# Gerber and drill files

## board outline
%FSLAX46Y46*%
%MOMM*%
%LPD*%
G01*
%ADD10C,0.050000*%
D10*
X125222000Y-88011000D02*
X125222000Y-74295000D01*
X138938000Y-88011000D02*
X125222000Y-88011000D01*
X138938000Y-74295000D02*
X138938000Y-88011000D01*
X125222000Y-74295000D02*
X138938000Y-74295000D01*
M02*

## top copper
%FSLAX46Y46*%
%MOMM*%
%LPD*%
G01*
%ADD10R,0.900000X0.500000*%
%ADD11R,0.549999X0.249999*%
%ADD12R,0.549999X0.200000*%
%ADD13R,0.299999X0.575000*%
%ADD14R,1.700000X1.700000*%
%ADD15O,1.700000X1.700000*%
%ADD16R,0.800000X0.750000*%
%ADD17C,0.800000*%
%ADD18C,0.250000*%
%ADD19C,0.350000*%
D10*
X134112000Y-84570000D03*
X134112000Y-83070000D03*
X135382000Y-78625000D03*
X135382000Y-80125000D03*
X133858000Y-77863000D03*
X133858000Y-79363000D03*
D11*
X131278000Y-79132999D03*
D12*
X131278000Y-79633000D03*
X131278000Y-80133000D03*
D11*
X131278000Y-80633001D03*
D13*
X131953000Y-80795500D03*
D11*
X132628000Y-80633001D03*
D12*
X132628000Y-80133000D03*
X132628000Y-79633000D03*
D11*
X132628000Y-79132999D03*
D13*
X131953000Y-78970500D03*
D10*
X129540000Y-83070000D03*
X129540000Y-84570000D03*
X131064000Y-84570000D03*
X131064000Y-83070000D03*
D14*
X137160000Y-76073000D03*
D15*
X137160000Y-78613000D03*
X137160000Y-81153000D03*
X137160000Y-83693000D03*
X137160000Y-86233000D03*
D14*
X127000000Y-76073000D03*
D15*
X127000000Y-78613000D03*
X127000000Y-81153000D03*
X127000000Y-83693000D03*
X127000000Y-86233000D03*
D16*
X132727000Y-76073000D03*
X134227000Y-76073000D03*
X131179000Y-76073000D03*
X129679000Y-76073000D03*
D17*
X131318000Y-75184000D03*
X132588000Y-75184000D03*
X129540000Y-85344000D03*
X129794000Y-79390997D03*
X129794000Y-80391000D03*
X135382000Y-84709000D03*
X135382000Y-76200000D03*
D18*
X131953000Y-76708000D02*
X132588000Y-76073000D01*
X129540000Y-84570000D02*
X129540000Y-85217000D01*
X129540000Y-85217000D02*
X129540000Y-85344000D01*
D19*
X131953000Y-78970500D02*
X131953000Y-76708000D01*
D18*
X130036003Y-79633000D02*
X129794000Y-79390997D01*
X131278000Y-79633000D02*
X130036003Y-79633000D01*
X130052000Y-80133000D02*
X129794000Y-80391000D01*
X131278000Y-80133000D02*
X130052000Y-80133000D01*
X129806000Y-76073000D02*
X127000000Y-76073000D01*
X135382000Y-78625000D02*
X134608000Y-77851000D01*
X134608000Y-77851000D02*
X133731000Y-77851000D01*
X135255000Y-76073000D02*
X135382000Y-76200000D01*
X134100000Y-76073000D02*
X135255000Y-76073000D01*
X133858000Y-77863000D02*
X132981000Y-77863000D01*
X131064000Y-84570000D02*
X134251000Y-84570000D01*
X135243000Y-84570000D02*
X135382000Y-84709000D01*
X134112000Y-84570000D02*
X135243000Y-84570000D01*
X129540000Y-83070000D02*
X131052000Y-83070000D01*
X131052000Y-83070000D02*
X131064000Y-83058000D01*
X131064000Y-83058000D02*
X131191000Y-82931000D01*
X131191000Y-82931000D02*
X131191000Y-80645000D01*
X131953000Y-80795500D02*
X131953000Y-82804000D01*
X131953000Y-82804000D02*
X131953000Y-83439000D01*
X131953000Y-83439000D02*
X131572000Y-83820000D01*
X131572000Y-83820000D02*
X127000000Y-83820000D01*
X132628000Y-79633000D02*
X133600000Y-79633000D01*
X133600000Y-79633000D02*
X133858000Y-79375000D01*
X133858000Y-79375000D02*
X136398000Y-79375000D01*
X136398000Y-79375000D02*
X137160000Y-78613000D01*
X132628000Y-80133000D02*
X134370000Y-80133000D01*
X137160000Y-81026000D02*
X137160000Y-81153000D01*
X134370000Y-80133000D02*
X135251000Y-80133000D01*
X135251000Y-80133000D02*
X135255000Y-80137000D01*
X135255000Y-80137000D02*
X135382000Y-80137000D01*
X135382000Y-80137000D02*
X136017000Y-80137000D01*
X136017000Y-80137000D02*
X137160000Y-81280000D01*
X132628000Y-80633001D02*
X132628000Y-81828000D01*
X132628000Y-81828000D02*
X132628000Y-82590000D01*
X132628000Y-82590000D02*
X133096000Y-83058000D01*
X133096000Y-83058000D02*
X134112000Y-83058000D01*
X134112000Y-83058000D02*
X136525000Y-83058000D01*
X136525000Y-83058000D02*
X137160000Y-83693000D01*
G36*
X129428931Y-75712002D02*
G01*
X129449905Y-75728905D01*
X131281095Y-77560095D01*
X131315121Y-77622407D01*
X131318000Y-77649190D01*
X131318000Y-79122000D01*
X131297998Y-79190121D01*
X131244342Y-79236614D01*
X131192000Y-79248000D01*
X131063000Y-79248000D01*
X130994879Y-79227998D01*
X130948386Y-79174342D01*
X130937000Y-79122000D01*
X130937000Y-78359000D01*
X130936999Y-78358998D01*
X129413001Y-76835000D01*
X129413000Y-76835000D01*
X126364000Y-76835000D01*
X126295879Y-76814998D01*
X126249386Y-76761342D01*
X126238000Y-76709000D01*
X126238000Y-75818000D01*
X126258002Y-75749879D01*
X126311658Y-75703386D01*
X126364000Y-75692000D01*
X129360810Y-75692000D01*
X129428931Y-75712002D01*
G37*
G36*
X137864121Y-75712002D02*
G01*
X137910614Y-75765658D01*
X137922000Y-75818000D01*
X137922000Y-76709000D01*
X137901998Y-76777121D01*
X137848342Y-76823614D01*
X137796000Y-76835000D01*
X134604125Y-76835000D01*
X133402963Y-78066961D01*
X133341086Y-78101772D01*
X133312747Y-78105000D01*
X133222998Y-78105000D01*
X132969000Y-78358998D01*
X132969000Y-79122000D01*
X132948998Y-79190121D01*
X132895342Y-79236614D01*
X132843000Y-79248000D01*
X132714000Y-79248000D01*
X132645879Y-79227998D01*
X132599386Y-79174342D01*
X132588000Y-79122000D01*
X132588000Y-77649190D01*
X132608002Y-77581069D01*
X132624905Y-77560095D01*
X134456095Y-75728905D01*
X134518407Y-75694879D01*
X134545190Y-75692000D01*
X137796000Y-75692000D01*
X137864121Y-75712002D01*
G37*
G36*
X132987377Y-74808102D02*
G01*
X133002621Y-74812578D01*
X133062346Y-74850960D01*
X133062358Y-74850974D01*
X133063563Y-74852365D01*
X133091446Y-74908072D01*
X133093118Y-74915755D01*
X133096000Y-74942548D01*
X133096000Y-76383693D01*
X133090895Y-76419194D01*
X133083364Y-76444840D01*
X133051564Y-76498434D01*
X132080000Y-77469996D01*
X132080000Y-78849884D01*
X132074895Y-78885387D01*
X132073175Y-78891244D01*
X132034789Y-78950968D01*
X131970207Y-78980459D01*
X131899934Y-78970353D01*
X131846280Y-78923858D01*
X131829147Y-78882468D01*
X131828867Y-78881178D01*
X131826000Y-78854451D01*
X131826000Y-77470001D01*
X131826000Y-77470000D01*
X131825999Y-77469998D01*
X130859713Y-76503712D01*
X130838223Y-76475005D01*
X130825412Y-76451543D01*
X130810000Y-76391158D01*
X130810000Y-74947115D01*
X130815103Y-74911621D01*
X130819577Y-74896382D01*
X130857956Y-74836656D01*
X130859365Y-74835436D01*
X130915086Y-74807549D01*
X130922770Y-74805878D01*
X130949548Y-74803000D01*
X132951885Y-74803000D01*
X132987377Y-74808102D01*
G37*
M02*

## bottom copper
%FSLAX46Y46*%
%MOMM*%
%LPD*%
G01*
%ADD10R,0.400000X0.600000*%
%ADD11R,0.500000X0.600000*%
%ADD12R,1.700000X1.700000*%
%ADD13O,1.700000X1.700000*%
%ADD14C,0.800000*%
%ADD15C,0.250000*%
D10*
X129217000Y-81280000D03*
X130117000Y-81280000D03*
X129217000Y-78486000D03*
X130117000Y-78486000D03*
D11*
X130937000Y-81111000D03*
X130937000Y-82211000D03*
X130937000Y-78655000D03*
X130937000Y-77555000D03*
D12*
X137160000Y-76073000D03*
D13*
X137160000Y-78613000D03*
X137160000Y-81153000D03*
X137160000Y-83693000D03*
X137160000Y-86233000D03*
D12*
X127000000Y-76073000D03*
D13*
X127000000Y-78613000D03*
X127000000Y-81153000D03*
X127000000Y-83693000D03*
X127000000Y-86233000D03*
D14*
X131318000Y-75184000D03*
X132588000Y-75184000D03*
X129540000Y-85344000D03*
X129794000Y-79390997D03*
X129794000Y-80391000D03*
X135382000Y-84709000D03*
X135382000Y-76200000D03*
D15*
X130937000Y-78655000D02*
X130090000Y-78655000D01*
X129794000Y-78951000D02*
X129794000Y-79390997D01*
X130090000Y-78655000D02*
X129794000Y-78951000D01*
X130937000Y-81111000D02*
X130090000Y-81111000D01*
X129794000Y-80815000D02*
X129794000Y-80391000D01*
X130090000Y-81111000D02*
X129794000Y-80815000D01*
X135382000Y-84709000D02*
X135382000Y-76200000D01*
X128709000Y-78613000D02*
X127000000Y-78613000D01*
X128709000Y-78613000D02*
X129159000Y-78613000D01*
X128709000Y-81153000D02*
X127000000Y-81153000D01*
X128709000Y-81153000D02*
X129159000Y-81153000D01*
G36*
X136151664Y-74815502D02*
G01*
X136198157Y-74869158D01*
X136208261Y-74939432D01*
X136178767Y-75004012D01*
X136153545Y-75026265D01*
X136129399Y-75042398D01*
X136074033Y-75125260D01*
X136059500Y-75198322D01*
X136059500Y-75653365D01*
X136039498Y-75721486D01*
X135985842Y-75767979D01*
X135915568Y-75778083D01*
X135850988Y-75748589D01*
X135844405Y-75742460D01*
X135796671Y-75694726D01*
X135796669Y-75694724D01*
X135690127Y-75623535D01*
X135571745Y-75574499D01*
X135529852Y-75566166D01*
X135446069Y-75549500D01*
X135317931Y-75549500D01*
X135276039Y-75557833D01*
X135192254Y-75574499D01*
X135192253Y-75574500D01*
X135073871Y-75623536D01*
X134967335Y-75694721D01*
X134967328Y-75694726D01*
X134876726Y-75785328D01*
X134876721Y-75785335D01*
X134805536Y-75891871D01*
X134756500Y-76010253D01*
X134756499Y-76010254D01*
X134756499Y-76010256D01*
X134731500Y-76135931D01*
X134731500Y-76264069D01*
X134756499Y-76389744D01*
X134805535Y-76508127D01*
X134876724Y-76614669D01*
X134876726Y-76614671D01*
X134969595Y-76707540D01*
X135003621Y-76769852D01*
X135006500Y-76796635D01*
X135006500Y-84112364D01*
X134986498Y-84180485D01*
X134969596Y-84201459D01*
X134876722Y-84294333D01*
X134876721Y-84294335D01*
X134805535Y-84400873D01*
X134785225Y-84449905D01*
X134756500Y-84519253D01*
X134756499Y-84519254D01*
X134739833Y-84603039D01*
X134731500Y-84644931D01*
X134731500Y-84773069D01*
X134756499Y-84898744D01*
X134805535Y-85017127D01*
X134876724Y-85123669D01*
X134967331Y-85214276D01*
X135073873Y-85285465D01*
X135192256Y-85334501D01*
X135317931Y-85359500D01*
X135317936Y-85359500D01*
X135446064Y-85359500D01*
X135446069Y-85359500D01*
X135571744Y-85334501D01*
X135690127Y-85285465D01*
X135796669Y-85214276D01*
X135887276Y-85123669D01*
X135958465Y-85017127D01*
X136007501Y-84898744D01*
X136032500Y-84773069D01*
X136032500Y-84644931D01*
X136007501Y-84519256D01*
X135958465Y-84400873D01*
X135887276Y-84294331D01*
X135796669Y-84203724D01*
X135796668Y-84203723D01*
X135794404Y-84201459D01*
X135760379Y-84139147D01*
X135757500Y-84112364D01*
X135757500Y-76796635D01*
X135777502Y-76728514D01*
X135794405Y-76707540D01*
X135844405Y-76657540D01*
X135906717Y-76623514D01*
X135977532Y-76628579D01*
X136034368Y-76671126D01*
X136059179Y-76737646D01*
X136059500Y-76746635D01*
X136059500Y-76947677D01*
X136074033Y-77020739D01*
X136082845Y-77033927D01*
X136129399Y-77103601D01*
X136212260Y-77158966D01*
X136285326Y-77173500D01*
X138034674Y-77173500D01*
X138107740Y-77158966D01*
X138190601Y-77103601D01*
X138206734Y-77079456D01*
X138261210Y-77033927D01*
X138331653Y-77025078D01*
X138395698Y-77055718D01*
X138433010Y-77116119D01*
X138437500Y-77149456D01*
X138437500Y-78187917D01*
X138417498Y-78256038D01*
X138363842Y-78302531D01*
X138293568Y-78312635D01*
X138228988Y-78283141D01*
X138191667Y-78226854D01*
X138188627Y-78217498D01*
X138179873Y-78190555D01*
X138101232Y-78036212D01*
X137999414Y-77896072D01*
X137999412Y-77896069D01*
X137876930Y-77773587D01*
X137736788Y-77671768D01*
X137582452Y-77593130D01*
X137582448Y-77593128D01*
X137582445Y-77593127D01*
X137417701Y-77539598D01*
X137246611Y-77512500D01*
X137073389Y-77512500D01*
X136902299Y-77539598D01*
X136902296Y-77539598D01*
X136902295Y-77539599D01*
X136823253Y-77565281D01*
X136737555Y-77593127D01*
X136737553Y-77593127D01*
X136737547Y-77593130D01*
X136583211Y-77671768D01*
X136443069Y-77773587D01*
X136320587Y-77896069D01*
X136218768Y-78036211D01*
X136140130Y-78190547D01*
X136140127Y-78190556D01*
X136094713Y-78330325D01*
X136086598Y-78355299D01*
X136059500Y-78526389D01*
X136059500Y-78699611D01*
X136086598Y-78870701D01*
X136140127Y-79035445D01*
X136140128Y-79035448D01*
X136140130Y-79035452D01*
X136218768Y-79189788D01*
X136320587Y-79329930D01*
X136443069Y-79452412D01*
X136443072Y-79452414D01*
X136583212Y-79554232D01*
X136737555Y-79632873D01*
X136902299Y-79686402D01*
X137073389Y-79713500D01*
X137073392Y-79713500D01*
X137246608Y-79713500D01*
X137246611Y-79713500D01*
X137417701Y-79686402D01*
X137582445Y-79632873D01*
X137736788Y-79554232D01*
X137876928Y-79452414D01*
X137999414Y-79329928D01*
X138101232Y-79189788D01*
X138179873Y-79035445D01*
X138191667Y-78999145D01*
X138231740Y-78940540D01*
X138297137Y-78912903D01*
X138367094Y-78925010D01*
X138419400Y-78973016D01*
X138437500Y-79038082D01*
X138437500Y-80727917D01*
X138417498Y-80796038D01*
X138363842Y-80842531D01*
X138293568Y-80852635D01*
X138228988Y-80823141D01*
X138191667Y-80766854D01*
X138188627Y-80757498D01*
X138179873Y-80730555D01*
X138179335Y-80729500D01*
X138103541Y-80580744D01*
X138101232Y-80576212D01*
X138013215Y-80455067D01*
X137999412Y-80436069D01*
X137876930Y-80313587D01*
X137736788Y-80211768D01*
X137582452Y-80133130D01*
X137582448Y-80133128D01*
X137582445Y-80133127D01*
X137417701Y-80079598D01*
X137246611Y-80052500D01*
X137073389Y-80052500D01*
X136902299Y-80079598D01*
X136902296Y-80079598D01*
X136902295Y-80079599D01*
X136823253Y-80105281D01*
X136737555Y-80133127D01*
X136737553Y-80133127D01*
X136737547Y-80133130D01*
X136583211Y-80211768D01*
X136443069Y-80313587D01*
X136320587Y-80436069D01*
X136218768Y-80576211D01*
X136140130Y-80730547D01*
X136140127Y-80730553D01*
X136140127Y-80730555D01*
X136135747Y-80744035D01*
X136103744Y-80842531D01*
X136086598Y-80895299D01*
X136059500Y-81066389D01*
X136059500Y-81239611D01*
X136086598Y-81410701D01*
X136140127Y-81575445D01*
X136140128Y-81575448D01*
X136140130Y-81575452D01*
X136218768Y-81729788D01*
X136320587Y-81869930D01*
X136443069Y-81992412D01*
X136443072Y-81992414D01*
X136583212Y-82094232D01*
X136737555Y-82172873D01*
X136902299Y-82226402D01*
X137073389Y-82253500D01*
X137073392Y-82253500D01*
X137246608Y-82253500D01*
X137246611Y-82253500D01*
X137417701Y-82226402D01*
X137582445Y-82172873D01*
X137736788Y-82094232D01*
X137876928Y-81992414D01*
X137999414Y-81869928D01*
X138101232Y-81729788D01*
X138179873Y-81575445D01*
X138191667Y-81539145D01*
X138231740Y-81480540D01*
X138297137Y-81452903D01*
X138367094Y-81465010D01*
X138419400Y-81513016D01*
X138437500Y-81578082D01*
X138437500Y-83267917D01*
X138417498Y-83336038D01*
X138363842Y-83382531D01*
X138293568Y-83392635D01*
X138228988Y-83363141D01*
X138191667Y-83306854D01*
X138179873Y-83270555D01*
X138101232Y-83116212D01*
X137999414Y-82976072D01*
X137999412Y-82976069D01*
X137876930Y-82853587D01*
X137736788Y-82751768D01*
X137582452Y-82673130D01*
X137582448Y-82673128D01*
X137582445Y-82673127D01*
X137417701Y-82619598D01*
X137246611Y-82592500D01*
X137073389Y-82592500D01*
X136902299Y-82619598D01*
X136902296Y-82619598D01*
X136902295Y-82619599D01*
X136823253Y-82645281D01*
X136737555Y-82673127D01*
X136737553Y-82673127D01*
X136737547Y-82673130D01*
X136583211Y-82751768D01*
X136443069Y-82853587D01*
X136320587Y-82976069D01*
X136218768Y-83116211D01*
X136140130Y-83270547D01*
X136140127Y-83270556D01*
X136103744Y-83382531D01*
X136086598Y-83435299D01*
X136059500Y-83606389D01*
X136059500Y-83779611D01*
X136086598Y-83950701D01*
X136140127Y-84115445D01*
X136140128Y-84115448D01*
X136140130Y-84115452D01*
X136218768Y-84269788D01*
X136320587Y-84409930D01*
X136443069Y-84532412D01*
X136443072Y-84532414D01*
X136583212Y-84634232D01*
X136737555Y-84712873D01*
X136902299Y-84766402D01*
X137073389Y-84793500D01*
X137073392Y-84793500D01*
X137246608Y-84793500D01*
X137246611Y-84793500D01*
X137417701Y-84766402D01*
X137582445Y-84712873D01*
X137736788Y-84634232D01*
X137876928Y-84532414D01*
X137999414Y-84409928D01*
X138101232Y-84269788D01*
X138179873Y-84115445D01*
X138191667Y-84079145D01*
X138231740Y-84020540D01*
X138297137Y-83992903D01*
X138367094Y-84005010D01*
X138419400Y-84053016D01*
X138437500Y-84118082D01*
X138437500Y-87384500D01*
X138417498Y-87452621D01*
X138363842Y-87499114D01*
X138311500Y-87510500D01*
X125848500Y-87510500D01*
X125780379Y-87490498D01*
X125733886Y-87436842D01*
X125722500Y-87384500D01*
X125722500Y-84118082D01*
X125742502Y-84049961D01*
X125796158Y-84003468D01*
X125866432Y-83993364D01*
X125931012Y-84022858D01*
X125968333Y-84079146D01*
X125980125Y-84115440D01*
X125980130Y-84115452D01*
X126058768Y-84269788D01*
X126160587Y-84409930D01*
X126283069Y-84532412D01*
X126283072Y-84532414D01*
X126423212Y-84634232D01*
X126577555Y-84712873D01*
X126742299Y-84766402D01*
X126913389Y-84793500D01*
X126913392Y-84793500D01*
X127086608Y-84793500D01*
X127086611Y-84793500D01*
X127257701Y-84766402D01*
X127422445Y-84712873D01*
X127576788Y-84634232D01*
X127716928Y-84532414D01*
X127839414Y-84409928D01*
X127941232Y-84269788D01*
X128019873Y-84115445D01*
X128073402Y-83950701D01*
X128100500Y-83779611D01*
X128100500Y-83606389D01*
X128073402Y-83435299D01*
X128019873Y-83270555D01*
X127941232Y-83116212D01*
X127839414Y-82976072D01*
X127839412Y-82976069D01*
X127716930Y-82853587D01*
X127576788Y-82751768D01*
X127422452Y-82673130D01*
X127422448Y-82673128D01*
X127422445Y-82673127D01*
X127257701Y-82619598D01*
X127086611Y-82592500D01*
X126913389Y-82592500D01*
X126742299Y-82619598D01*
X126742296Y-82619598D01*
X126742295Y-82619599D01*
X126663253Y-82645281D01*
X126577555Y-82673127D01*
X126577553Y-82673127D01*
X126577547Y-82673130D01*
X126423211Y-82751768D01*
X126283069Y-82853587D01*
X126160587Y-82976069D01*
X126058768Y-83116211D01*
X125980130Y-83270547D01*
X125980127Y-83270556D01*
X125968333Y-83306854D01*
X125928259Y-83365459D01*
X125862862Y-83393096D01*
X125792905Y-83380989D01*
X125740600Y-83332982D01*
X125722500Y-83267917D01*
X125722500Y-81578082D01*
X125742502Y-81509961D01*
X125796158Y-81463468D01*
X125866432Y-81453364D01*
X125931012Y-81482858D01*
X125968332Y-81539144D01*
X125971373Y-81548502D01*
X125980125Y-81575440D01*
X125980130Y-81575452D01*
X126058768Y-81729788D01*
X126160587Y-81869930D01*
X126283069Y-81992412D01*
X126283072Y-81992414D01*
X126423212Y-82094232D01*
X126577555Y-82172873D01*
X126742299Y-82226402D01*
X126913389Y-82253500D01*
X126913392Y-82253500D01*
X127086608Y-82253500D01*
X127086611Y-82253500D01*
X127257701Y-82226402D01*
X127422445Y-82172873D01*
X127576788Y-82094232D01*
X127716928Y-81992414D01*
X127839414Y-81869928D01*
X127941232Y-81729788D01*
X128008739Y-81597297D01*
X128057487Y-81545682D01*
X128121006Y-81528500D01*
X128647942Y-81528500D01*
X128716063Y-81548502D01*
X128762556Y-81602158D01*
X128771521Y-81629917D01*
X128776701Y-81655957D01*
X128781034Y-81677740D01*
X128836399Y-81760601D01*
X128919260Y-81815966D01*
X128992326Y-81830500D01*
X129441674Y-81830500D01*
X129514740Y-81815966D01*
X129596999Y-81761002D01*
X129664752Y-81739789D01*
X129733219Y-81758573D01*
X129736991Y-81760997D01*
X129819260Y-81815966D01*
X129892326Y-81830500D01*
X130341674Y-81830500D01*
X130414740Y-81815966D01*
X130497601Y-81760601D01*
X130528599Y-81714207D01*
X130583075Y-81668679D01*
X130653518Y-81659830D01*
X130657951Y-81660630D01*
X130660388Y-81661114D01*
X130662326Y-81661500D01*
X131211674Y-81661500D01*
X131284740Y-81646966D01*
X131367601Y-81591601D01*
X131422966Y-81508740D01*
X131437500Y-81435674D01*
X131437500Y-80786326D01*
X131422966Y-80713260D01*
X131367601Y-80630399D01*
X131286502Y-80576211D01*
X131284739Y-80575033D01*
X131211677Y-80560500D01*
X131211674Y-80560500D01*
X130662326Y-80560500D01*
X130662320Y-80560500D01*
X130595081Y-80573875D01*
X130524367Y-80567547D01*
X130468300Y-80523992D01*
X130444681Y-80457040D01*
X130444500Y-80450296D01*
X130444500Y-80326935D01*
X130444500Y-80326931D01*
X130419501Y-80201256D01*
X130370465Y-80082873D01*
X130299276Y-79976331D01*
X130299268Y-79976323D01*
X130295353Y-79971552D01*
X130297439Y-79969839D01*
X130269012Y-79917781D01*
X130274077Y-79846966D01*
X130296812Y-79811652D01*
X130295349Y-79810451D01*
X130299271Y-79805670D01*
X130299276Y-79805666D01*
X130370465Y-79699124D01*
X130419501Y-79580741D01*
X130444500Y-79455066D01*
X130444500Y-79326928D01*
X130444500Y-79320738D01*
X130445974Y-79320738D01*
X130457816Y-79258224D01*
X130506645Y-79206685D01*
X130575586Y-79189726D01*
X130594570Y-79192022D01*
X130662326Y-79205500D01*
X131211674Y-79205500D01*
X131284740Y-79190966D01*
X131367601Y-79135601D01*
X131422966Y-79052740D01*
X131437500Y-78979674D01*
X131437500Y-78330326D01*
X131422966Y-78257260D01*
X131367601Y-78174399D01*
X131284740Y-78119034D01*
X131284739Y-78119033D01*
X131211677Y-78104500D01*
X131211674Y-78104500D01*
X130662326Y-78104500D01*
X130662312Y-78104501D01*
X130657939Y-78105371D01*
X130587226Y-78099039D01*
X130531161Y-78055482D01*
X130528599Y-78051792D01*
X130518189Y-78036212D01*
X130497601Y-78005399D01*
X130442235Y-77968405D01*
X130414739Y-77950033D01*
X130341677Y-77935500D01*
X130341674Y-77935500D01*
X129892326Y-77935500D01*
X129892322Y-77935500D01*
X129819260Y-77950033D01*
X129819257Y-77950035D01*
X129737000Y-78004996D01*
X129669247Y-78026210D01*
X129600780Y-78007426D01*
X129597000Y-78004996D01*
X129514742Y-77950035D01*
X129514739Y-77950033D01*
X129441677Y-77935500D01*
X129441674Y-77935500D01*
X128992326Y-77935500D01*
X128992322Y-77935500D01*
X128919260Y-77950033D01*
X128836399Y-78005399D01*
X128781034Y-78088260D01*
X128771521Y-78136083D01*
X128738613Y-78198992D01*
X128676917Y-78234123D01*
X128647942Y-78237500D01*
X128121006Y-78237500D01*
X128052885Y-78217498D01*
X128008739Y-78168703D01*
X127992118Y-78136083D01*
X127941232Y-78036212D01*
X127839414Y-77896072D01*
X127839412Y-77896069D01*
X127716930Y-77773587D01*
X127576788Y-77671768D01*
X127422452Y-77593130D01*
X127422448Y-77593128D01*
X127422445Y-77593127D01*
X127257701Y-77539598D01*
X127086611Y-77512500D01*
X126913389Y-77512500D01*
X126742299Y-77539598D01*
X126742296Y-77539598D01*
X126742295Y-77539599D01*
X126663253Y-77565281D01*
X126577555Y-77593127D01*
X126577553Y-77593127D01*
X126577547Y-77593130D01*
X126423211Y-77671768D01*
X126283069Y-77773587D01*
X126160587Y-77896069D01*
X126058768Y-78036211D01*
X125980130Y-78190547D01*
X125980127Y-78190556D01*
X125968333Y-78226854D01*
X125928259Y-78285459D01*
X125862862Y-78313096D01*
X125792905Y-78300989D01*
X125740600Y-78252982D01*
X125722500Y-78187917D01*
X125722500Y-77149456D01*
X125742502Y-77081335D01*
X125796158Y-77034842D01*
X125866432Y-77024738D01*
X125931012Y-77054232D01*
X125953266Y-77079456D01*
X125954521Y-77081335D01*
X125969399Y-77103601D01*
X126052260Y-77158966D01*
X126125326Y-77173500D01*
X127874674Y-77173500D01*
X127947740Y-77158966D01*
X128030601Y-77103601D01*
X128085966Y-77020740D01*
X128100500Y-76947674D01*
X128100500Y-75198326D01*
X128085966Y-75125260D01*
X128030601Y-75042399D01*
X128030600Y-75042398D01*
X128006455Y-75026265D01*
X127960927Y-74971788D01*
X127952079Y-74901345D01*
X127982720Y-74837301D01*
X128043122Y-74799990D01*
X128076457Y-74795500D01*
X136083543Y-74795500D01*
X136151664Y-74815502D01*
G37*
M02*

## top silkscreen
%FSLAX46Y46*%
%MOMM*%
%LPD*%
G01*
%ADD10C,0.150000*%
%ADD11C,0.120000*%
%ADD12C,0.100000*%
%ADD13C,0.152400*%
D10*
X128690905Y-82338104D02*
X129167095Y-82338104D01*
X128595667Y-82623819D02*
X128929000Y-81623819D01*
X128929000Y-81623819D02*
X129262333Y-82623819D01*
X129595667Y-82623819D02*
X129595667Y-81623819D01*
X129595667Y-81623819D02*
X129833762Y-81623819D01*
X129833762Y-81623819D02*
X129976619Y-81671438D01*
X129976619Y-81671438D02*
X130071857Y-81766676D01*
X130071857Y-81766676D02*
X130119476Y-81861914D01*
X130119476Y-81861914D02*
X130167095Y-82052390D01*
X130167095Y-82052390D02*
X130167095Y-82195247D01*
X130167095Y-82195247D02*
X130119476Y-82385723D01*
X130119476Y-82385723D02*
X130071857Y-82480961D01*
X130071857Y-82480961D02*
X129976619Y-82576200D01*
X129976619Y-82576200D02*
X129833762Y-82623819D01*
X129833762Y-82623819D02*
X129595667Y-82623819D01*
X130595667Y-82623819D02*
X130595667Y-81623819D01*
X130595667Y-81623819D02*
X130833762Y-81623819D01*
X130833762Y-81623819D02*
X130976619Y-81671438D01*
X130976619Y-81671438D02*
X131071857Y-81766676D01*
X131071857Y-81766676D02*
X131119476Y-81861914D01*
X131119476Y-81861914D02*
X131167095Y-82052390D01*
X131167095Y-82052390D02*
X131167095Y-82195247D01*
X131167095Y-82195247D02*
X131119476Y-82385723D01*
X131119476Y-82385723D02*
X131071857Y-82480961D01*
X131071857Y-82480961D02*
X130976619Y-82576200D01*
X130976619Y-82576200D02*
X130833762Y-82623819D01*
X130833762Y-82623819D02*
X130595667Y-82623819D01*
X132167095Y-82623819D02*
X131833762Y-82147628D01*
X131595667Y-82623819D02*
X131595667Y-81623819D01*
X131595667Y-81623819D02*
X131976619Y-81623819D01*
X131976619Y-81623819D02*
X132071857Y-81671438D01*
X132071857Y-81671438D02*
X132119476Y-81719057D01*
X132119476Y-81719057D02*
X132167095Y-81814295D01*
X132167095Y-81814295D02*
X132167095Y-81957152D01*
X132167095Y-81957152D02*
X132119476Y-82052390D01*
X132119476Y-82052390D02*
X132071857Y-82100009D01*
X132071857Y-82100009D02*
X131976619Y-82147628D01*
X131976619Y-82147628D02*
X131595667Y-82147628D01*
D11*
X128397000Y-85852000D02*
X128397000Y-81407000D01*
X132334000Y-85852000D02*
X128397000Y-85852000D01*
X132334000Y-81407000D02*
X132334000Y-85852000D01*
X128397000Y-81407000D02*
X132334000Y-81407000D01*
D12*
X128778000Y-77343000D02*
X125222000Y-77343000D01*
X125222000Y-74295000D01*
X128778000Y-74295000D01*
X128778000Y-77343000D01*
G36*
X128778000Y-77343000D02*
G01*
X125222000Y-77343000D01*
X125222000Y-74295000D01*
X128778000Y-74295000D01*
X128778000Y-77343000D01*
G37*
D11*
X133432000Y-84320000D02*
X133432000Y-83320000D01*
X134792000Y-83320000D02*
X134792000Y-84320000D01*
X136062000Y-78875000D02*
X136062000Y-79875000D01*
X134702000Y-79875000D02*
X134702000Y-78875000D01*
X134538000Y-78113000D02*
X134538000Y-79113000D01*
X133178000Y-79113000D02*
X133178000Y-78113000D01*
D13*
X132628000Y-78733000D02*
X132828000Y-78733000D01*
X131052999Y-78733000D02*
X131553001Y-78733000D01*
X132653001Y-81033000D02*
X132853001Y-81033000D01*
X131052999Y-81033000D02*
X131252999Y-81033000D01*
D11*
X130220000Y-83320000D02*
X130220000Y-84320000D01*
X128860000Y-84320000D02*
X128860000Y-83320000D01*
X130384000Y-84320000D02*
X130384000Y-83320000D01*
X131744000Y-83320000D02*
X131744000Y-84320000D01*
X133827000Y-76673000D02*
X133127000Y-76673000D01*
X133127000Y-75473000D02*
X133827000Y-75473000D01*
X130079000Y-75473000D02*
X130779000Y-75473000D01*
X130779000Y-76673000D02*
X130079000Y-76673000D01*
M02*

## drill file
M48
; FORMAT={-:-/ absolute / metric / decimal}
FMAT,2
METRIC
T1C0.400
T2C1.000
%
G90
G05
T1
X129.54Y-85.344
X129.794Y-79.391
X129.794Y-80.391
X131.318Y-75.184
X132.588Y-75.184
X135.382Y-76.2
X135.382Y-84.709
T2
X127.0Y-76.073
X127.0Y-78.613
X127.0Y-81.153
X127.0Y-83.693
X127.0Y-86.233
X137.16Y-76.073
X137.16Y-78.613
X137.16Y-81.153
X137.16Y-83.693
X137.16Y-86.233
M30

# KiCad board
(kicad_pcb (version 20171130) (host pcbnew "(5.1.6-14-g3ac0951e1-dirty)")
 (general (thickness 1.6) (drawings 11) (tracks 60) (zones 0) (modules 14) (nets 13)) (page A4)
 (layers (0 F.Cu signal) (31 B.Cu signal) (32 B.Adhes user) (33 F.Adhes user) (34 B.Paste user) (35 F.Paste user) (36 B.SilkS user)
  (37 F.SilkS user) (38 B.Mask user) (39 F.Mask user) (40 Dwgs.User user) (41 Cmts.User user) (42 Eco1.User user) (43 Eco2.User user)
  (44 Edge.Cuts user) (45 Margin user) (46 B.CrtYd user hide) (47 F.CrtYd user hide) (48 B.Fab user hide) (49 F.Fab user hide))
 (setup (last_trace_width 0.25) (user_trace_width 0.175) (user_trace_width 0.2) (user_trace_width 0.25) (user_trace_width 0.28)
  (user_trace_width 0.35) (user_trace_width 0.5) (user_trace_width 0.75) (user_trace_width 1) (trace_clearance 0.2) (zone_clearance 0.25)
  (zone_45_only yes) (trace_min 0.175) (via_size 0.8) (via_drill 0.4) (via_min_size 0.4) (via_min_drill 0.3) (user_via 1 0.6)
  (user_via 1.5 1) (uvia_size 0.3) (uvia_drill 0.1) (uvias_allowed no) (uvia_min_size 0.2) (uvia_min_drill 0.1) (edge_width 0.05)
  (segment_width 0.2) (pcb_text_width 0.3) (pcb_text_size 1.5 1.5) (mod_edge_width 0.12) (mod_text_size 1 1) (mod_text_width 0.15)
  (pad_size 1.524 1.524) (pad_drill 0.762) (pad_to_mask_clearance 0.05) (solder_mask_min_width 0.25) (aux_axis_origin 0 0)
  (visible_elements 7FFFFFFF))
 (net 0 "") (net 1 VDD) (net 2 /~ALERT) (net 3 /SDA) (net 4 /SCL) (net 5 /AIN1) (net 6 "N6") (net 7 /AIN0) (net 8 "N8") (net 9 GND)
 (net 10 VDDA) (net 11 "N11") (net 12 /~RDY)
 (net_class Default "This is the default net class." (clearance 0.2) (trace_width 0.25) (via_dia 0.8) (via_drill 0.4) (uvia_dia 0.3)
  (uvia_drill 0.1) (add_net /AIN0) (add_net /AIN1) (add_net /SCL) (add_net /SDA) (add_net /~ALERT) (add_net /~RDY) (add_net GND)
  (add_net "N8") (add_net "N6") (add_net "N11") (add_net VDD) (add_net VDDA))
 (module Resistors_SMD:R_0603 (layer F.Cu) (at 134.112 83.82 90)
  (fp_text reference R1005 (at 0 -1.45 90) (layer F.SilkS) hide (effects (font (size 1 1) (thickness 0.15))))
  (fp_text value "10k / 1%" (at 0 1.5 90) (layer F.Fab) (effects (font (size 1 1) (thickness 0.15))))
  (fp_line (start -0.5 -0.68) (end 0.5 -0.68) (layer F.SilkS) (width 0.12))
  (fp_line (start 0.5 0.68) (end -0.5 0.68) (layer F.SilkS) (width 0.12))
  (pad 1 smd rect (at -0.75 0 90) (size 0.5 0.9) (layers F.Cu F.Paste F.Mask) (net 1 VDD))
  (pad 2 smd rect (at 0.75 0 90) (size 0.5 0.9) (layers F.Cu F.Paste F.Mask) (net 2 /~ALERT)))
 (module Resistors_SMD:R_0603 (layer F.Cu) (at 135.382 79.375 270)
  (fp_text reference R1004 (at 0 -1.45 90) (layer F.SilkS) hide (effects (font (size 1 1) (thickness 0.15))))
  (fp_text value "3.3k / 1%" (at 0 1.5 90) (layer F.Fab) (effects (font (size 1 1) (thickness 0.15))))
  (fp_line (start -0.5 -0.68) (end 0.5 -0.68) (layer F.SilkS) (width 0.12))
  (fp_line (start 0.5 0.68) (end -0.5 0.68) (layer F.SilkS) (width 0.12))
  (pad 1 smd rect (at -0.75 0 270) (size 0.5 0.9) (layers F.Cu F.Paste F.Mask) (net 1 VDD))
  (pad 2 smd rect (at 0.75 0 270) (size 0.5 0.9) (layers F.Cu F.Paste F.Mask) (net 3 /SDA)))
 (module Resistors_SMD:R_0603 (layer F.Cu) (at 133.858 78.613 270)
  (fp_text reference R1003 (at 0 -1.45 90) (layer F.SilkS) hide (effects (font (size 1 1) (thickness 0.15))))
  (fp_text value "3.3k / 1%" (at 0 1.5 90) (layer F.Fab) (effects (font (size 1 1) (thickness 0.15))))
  (fp_line (start -0.5 -0.68) (end 0.5 -0.68) (layer F.SilkS) (width 0.12))
  (fp_line (start 0.5 0.68) (end -0.5 0.68) (layer F.SilkS) (width 0.12))
  (pad 1 smd rect (at -0.75 0 270) (size 0.5 0.9) (layers F.Cu F.Paste F.Mask) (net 1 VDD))
  (pad 2 smd rect (at 0.75 0 270) (size 0.5 0.9) (layers F.Cu F.Paste F.Mask) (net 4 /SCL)))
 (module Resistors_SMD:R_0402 (layer B.Cu) (at 129.667 81.28)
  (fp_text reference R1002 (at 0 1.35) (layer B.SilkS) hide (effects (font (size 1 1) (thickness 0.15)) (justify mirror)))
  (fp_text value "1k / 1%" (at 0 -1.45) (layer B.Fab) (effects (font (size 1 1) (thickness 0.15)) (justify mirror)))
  (pad 1 smd rect (at -0.45 0) (size 0.4 0.6) (layers B.Cu B.Paste B.Mask) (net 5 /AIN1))
  (pad 2 smd rect (at 0.45 0) (size 0.4 0.6) (layers B.Cu B.Paste B.Mask) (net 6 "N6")))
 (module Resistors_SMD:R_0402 (layer B.Cu) (at 129.667 78.486)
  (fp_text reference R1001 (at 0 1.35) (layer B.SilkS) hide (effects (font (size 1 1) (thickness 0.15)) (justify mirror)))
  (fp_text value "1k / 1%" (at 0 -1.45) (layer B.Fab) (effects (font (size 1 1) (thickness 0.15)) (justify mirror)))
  (pad 1 smd rect (at -0.45 0) (size 0.4 0.6) (layers B.Cu B.Paste B.Mask) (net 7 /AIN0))
  (pad 2 smd rect (at 0.45 0) (size 0.4 0.6) (layers B.Cu B.Paste B.Mask) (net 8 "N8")))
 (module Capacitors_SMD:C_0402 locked (layer B.Cu) (at 130.937 81.661 270)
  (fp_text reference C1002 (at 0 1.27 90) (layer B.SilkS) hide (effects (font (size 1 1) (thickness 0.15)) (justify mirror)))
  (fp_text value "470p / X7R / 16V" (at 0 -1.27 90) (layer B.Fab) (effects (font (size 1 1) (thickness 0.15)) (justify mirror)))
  (pad 1 smd rect (at -0.55 0 270) (size 0.6 0.5) (layers B.Cu B.Paste B.Mask) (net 6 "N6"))
  (pad 2 smd rect (at 0.55 0 270) (size 0.6 0.5) (layers B.Cu B.Paste B.Mask) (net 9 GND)))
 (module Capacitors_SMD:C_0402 (layer B.Cu) (at 130.937 78.105 90)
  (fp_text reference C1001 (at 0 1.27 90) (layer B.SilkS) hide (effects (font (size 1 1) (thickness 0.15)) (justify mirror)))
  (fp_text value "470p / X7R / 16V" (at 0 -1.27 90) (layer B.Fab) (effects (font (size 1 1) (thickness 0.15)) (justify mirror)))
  (pad 1 smd rect (at -0.55 0 90) (size 0.6 0.5) (layers B.Cu B.Paste B.Mask) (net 8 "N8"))
  (pad 2 smd rect (at 0.55 0 90) (size 0.6 0.5) (layers B.Cu B.Paste B.Mask) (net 9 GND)))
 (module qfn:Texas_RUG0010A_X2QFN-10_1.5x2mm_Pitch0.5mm (layer F.Cu) (at 131.953 79.883)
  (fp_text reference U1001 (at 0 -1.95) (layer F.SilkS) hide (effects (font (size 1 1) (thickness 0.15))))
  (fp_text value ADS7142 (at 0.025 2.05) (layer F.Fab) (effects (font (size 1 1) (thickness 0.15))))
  (fp_line (start 0.675 -1.15) (end 0.875 -1.15) (layer F.SilkS) (width 0.1524))
  (fp_line (start -0.900001 -1.15) (end -0.399999 -1.15) (layer F.SilkS) (width 0.1524))
  (fp_line (start 0.700001 1.15) (end 0.900001 1.15) (layer F.SilkS) (width 0.1524))
  (fp_line (start -0.900001 1.15) (end -0.700001 1.15) (layer F.SilkS) (width 0.1524))
  (pad 1 smd rect (at -0.675 -0.750001 90) (size 0.249999 0.549999) (layers F.Cu F.Paste F.Mask) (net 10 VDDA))
  (pad 2 smd rect (at -0.675 -0.25 90) (size 0.2 0.549999) (layers F.Cu F.Paste F.Mask) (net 8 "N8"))
  (pad 3 smd rect (at -0.675 0.25 90) (size 0.2 0.549999) (layers F.Cu F.Paste F.Mask) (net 6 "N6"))
  (pad 4 smd rect (at -0.675 0.750001 90) (size 0.249999 0.549999) (layers F.Cu F.Paste F.Mask) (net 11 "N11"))
  (pad 5 smd rect (at 0 0.9125 90) (size 0.575 0.299999) (layers F.Cu F.Paste F.Mask) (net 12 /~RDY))
  (pad 6 smd rect (at 0.675 0.750001 90) (size 0.249999 0.549999) (layers F.Cu F.Paste F.Mask) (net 2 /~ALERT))
  (pad 7 smd rect (at 0.675 0.25 90) (size 0.2 0.549999) (layers F.Cu F.Paste F.Mask) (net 3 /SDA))
  (pad 8 smd rect (at 0.675 -0.25 90) (size 0.2 0.549999) (layers F.Cu F.Paste F.Mask) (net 4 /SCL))
  (pad 9 smd rect (at 0.675 -0.750001 90) (size 0.249999 0.549999) (layers F.Cu F.Paste F.Mask) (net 1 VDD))
  (pad 10 smd rect (at 0 -0.9125 90) (size 0.575 0.299999) (layers F.Cu F.Paste F.Mask) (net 9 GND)))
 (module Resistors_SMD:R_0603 (layer F.Cu) (at 129.54 83.82 270)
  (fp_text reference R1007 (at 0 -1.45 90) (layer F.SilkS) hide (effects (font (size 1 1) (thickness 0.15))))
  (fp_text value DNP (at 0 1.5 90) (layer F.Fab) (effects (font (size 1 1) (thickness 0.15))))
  (fp_line (start -0.5 -0.68) (end 0.5 -0.68) (layer F.SilkS) (width 0.12))
  (fp_line (start 0.5 0.68) (end -0.5 0.68) (layer F.SilkS) (width 0.12))
  (pad 1 smd rect (at -0.75 0 270) (size 0.5 0.9) (layers F.Cu F.Paste F.Mask) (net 11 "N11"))
  (pad 2 smd rect (at 0.75 0 270) (size 0.5 0.9) (layers F.Cu F.Paste F.Mask) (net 9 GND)))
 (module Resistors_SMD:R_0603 (layer F.Cu) (at 131.064 83.82 90)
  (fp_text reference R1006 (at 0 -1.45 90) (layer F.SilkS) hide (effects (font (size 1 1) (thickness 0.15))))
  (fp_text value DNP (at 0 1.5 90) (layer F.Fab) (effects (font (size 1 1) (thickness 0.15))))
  (fp_line (start -0.5 -0.68) (end 0.5 -0.68) (layer F.SilkS) (width 0.12))
  (fp_line (start 0.5 0.68) (end -0.5 0.68) (layer F.SilkS) (width 0.12))
  (pad 1 smd rect (at -0.75 0 90) (size 0.5 0.9) (layers F.Cu F.Paste F.Mask) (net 1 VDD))
  (pad 2 smd rect (at 0.75 0 90) (size 0.5 0.9) (layers F.Cu F.Paste F.Mask) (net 11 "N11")))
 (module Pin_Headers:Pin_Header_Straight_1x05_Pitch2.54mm (layer B.Cu) (at 137.16 76.073 180)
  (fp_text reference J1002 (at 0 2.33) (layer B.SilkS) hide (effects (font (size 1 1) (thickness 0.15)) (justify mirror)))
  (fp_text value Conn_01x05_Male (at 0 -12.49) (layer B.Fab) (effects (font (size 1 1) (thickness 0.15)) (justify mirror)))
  (pad 1 thru_hole rect (at 0 0 180) (size 1.7 1.7) (drill 1) (layers *.Cu *.Mask) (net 1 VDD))
  (pad 2 thru_hole oval (at 0 -2.54 180) (size 1.7 1.7) (drill 1) (layers *.Cu *.Mask) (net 4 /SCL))
  (pad 3 thru_hole oval (at 0 -5.08 180) (size 1.7 1.7) (drill 1) (layers *.Cu *.Mask) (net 3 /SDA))
  (pad 4 thru_hole oval (at 0 -7.62 180) (size 1.7 1.7) (drill 1) (layers *.Cu *.Mask) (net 2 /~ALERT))
  (pad 5 thru_hole oval (at 0 -10.16 180) (size 1.7 1.7) (drill 1) (layers *.Cu *.Mask) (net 9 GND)))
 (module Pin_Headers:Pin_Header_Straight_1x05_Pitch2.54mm (layer B.Cu) (at 127 76.073 180)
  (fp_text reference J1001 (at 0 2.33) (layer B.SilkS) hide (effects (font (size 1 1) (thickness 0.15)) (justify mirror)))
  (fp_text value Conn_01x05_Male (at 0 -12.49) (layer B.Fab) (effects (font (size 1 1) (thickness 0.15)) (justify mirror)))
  (pad 1 thru_hole rect (at 0 0 180) (size 1.7 1.7) (drill 1) (layers *.Cu *.Mask) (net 10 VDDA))
  (pad 2 thru_hole oval (at 0 -2.54 180) (size 1.7 1.7) (drill 1) (layers *.Cu *.Mask) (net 7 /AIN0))
  (pad 3 thru_hole oval (at 0 -5.08 180) (size 1.7 1.7) (drill 1) (layers *.Cu *.Mask) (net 5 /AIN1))
  (pad 4 thru_hole oval (at 0 -7.62 180) (size 1.7 1.7) (drill 1) (layers *.Cu *.Mask) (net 12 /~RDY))
  (pad 5 thru_hole oval (at 0 -10.16 180) (size 1.7 1.7) (drill 1) (layers *.Cu *.Mask) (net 9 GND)))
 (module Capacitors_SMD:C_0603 (layer F.Cu) (at 133.477 76.073 180)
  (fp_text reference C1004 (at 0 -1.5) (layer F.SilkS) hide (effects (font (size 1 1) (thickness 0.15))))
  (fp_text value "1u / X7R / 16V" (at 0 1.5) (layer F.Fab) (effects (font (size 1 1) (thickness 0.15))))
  (fp_line (start -0.35 -0.6) (end 0.35 -0.6) (layer F.SilkS) (width 0.12))
  (fp_line (start 0.35 0.6) (end -0.35 0.6) (layer F.SilkS) (width 0.12))
  (pad 2 smd rect (at 0.75 0 180) (size 0.8 0.75) (layers F.Cu F.Paste F.Mask) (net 9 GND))
  (pad 1 smd rect (at -0.75 0 180) (size 0.8 0.75) (layers F.Cu F.Paste F.Mask) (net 1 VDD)))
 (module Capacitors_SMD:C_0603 (layer F.Cu) (at 130.429 76.073)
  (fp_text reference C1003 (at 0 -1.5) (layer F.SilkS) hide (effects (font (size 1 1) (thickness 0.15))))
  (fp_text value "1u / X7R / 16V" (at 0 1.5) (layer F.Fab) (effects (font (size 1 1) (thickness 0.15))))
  (fp_line (start -0.35 -0.6) (end 0.35 -0.6) (layer F.SilkS) (width 0.12))
  (fp_line (start 0.35 0.6) (end -0.35 0.6) (layer F.SilkS) (width 0.12))
  (pad 2 smd rect (at 0.75 0) (size 0.8 0.75) (layers F.Cu F.Paste F.Mask) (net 9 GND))
  (pad 1 smd rect (at -0.75 0) (size 0.8 0.75) (layers F.Cu F.Paste F.Mask) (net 10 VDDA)))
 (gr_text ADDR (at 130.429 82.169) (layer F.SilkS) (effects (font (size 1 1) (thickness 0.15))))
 (gr_line (start 128.397 85.852) (end 128.397 81.407) (layer F.SilkS) (width 0.12))
 (gr_line (start 132.334 85.852) (end 128.397 85.852) (layer F.SilkS) (width 0.12))
 (gr_line (start 132.334 81.407) (end 132.334 85.852) (layer F.SilkS) (width 0.12))
 (gr_line (start 128.397 81.407) (end 132.334 81.407) (layer F.SilkS) (width 0.12))
 (gr_poly (pts (xy 128.778 77.343) (xy 125.222 77.343) (xy 125.222 74.295) (xy 128.778 74.295)) (layer F.SilkS) (width 0.1))
 (gr_line (start 125.222 88.011) (end 125.222 74.295) (layer Edge.Cuts) (width 0.05))
 (gr_line (start 138.938 88.011) (end 125.222 88.011) (layer Edge.Cuts) (width 0.05))
 (gr_line (start 138.938 74.295) (end 138.938 88.011) (layer Edge.Cuts) (width 0.05))
 (gr_line (start 125.222 74.295) (end 138.938 74.295) (layer Edge.Cuts) (width 0.05))
 (segment (start 131.953 76.708) (end 132.588 76.073) (width 0.25) (layer F.Cu) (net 9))
 (via (at 131.318 75.184) (size 0.8) (drill 0.4) (layers F.Cu B.Cu) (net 9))
 (via (at 132.588 75.184) (size 0.8) (drill 0.4) (layers F.Cu B.Cu) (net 9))
 (segment (start 129.54 84.57) (end 129.54 85.217) (width 0.25) (layer F.Cu) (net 9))
 (via (at 129.54 85.344) (size 0.8) (drill 0.4) (layers F.Cu B.Cu) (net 9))
 (segment (start 129.54 85.217) (end 129.54 85.344) (width 0.25) (layer F.Cu) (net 9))
 (segment (start 131.953 78.9705) (end 131.953 76.708) (width 0.35) (layer F.Cu) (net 9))
 (via (at 129.794 79.390997) (size 0.8) (drill 0.4) (layers F.Cu B.Cu) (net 8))
 (segment (start 130.036003 79.633) (end 129.794 79.390997) (width 0.25) (layer F.Cu) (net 8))
 (segment (start 131.278 79.633) (end 130.036003 79.633) (width 0.25) (layer F.Cu) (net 8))
 (segment (start 130.937 78.655) (end 130.09 78.655) (width 0.25) (layer B.Cu) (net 8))
 (segment (start 129.794 78.951) (end 129.794 79.390997) (width 0.25) (layer B.Cu) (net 8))
 (segment (start 130.09 78.655) (end 129.794 78.951) (width 0.25) (layer B.Cu) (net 8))
 (via (at 129.794 80.391) (size 0.8) (drill 0.4) (layers F.Cu B.Cu) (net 6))
 (segment (start 130.052 80.133) (end 129.794 80.391) (width 0.25) (layer F.Cu) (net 6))
 (segment (start 131.278 80.133) (end 130.052 80.133) (width 0.25) (layer F.Cu) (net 6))
 (segment (start 130.937 81.111) (end 130.09 81.111) (width 0.25) (layer B.Cu) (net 6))
 (segment (start 129.794 80.815) (end 129.794 80.391) (width 0.25) (layer B.Cu) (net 6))
 (segment (start 130.09 81.111) (end 129.794 80.815) (width 0.25) (layer B.Cu) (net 6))
 (segment (start 129.806 76.073) (end 127 76.073) (width 0.25) (layer F.Cu) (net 10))
 (via (at 135.382 84.709) (size 0.8) (drill 0.4) (layers F.Cu B.Cu) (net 1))
 (segment (start 135.382 84.709) (end 135.382 76.2) (width 0.25) (layer B.Cu) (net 1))
 (via (at 135.382 76.2) (size 0.8) (drill 0.4) (layers F.Cu B.Cu) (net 1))
 (segment (start 135.382 78.625) (end 134.608 77.851) (width 0.25) (layer F.Cu) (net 1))
 (segment (start 134.608 77.851) (end 133.731 77.851) (width 0.25) (layer F.Cu) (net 1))
 (segment (start 135.255 76.073) (end 135.382 76.2) (width 0.25) (layer F.Cu) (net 1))
 (segment (start 134.1 76.073) (end 135.255 76.073) (width 0.25) (layer F.Cu) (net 1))
 (segment (start 133.858 77.863) (end 132.981 77.863) (width 0.25) (layer F.Cu) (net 1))
 (segment (start 131.064 84.57) (end 134.251 84.57) (width 0.25) (layer F.Cu) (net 1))
 (segment (start 135.243 84.57) (end 135.382 84.709) (width 0.25) (layer F.Cu) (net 1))
 (segment (start 134.112 84.57) (end 135.243 84.57) (width 0.25) (layer F.Cu) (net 1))
 (segment (start 129.54 83.07) (end 131.052 83.07) (width 0.25) (layer F.Cu) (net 11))
 (segment (start 131.052 83.07) (end 131.064 83.058) (width 0.25) (layer F.Cu) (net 11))
 (segment (start 131.064 83.058) (end 131.191 82.931) (width 0.25) (layer F.Cu) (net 11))
 (segment (start 131.191 82.931) (end 131.191 80.645) (width 0.25) (layer F.Cu) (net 11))
 (segment (start 128.709 78.613) (end 127 78.613) (width 0.25) (layer B.Cu) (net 7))
 (segment (start 128.709 78.613) (end 129.159 78.613) (width 0.25) (layer B.Cu) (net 7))
 (segment (start 128.709 81.153) (end 127 81.153) (width 0.25) (layer B.Cu) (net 5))
 (segment (start 128.709 81.153) (end 129.159 81.153) (width 0.25) (layer B.Cu) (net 5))
 (segment (start 131.953 80.7955) (end 131.953 82.804) (width 0.25) (layer F.Cu) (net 12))
 (segment (start 131.953 82.804) (end 131.953 83.439) (width 0.25) (layer F.Cu) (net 12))
 (segment (start 131.953 83.439) (end 131.572 83.82) (width 0.25) (layer F.Cu) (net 12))
 (segment (start 131.572 83.82) (end 127 83.82) (width 0.25) (layer F.Cu) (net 12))
 (segment (start 132.628 79.633) (end 133.6 79.633) (width 0.25) (layer F.Cu) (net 4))
 (segment (start 133.6 79.633) (end 133.858 79.375) (width 0.25) (layer F.Cu) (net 4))
 (segment (start 133.858 79.375) (end 136.398 79.375) (width 0.25) (layer F.Cu) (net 4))
 (segment (start 136.398 79.375) (end 137.16 78.613) (width 0.25) (layer F.Cu) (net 4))
 (segment (start 132.628 80.133) (end 134.37 80.133) (width 0.25) (layer F.Cu) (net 3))
 (segment (start 137.16 81.026) (end 137.16 81.153) (width 0.25) (layer F.Cu) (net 3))
 (segment (start 134.37 80.133) (end 135.251 80.133) (width 0.25) (layer F.Cu) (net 3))
 (segment (start 135.251 80.133) (end 135.255 80.137) (width 0.25) (layer F.Cu) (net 3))
 (segment (start 135.255 80.137) (end 135.382 80.137) (width 0.25) (layer F.Cu) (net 3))
 (segment (start 135.382 80.137) (end 136.017 80.137) (width 0.25) (layer F.Cu) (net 3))
 (segment (start 136.017 80.137) (end 137.16 81.28) (width 0.25) (layer F.Cu) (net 3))
 (segment (start 132.628 80.633001) (end 132.628 81.828) (width 0.25) (layer F.Cu) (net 2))
 (segment (start 132.628 81.828) (end 132.628 82.59) (width 0.25) (layer F.Cu) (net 2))
 (segment (start 132.628 82.59) (end 133.096 83.058) (width 0.25) (layer F.Cu) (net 2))
 (segment (start 133.096 83.058) (end 134.112 83.058) (width 0.25) (layer F.Cu) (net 2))
 (segment (start 134.112 83.058) (end 136.525 83.058) (width 0.25) (layer F.Cu) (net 2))
 (segment (start 136.525 83.058) (end 137.16 83.693) (width 0.25) (layer F.Cu) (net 2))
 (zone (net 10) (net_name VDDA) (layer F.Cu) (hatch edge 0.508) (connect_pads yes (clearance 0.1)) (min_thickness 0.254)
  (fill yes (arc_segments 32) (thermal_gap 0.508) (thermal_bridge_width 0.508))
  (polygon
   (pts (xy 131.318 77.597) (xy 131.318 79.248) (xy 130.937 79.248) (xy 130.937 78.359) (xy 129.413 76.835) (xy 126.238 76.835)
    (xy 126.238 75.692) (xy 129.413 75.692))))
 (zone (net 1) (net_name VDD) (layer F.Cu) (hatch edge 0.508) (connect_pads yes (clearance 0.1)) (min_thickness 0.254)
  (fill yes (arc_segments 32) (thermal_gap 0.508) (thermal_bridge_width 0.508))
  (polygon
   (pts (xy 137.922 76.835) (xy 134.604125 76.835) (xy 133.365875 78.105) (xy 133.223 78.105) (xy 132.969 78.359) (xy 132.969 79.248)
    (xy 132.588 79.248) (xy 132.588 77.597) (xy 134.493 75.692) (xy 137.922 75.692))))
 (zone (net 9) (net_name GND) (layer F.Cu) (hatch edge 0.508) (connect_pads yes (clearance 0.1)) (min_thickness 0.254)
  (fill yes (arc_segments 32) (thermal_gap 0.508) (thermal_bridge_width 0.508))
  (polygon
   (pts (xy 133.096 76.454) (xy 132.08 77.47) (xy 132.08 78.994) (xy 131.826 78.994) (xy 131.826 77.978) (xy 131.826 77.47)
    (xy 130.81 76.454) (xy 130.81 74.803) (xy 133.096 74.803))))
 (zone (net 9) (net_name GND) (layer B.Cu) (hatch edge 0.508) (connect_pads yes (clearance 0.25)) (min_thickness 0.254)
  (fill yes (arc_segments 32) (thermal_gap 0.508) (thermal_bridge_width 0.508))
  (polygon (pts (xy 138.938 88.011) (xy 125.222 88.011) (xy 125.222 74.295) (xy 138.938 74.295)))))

